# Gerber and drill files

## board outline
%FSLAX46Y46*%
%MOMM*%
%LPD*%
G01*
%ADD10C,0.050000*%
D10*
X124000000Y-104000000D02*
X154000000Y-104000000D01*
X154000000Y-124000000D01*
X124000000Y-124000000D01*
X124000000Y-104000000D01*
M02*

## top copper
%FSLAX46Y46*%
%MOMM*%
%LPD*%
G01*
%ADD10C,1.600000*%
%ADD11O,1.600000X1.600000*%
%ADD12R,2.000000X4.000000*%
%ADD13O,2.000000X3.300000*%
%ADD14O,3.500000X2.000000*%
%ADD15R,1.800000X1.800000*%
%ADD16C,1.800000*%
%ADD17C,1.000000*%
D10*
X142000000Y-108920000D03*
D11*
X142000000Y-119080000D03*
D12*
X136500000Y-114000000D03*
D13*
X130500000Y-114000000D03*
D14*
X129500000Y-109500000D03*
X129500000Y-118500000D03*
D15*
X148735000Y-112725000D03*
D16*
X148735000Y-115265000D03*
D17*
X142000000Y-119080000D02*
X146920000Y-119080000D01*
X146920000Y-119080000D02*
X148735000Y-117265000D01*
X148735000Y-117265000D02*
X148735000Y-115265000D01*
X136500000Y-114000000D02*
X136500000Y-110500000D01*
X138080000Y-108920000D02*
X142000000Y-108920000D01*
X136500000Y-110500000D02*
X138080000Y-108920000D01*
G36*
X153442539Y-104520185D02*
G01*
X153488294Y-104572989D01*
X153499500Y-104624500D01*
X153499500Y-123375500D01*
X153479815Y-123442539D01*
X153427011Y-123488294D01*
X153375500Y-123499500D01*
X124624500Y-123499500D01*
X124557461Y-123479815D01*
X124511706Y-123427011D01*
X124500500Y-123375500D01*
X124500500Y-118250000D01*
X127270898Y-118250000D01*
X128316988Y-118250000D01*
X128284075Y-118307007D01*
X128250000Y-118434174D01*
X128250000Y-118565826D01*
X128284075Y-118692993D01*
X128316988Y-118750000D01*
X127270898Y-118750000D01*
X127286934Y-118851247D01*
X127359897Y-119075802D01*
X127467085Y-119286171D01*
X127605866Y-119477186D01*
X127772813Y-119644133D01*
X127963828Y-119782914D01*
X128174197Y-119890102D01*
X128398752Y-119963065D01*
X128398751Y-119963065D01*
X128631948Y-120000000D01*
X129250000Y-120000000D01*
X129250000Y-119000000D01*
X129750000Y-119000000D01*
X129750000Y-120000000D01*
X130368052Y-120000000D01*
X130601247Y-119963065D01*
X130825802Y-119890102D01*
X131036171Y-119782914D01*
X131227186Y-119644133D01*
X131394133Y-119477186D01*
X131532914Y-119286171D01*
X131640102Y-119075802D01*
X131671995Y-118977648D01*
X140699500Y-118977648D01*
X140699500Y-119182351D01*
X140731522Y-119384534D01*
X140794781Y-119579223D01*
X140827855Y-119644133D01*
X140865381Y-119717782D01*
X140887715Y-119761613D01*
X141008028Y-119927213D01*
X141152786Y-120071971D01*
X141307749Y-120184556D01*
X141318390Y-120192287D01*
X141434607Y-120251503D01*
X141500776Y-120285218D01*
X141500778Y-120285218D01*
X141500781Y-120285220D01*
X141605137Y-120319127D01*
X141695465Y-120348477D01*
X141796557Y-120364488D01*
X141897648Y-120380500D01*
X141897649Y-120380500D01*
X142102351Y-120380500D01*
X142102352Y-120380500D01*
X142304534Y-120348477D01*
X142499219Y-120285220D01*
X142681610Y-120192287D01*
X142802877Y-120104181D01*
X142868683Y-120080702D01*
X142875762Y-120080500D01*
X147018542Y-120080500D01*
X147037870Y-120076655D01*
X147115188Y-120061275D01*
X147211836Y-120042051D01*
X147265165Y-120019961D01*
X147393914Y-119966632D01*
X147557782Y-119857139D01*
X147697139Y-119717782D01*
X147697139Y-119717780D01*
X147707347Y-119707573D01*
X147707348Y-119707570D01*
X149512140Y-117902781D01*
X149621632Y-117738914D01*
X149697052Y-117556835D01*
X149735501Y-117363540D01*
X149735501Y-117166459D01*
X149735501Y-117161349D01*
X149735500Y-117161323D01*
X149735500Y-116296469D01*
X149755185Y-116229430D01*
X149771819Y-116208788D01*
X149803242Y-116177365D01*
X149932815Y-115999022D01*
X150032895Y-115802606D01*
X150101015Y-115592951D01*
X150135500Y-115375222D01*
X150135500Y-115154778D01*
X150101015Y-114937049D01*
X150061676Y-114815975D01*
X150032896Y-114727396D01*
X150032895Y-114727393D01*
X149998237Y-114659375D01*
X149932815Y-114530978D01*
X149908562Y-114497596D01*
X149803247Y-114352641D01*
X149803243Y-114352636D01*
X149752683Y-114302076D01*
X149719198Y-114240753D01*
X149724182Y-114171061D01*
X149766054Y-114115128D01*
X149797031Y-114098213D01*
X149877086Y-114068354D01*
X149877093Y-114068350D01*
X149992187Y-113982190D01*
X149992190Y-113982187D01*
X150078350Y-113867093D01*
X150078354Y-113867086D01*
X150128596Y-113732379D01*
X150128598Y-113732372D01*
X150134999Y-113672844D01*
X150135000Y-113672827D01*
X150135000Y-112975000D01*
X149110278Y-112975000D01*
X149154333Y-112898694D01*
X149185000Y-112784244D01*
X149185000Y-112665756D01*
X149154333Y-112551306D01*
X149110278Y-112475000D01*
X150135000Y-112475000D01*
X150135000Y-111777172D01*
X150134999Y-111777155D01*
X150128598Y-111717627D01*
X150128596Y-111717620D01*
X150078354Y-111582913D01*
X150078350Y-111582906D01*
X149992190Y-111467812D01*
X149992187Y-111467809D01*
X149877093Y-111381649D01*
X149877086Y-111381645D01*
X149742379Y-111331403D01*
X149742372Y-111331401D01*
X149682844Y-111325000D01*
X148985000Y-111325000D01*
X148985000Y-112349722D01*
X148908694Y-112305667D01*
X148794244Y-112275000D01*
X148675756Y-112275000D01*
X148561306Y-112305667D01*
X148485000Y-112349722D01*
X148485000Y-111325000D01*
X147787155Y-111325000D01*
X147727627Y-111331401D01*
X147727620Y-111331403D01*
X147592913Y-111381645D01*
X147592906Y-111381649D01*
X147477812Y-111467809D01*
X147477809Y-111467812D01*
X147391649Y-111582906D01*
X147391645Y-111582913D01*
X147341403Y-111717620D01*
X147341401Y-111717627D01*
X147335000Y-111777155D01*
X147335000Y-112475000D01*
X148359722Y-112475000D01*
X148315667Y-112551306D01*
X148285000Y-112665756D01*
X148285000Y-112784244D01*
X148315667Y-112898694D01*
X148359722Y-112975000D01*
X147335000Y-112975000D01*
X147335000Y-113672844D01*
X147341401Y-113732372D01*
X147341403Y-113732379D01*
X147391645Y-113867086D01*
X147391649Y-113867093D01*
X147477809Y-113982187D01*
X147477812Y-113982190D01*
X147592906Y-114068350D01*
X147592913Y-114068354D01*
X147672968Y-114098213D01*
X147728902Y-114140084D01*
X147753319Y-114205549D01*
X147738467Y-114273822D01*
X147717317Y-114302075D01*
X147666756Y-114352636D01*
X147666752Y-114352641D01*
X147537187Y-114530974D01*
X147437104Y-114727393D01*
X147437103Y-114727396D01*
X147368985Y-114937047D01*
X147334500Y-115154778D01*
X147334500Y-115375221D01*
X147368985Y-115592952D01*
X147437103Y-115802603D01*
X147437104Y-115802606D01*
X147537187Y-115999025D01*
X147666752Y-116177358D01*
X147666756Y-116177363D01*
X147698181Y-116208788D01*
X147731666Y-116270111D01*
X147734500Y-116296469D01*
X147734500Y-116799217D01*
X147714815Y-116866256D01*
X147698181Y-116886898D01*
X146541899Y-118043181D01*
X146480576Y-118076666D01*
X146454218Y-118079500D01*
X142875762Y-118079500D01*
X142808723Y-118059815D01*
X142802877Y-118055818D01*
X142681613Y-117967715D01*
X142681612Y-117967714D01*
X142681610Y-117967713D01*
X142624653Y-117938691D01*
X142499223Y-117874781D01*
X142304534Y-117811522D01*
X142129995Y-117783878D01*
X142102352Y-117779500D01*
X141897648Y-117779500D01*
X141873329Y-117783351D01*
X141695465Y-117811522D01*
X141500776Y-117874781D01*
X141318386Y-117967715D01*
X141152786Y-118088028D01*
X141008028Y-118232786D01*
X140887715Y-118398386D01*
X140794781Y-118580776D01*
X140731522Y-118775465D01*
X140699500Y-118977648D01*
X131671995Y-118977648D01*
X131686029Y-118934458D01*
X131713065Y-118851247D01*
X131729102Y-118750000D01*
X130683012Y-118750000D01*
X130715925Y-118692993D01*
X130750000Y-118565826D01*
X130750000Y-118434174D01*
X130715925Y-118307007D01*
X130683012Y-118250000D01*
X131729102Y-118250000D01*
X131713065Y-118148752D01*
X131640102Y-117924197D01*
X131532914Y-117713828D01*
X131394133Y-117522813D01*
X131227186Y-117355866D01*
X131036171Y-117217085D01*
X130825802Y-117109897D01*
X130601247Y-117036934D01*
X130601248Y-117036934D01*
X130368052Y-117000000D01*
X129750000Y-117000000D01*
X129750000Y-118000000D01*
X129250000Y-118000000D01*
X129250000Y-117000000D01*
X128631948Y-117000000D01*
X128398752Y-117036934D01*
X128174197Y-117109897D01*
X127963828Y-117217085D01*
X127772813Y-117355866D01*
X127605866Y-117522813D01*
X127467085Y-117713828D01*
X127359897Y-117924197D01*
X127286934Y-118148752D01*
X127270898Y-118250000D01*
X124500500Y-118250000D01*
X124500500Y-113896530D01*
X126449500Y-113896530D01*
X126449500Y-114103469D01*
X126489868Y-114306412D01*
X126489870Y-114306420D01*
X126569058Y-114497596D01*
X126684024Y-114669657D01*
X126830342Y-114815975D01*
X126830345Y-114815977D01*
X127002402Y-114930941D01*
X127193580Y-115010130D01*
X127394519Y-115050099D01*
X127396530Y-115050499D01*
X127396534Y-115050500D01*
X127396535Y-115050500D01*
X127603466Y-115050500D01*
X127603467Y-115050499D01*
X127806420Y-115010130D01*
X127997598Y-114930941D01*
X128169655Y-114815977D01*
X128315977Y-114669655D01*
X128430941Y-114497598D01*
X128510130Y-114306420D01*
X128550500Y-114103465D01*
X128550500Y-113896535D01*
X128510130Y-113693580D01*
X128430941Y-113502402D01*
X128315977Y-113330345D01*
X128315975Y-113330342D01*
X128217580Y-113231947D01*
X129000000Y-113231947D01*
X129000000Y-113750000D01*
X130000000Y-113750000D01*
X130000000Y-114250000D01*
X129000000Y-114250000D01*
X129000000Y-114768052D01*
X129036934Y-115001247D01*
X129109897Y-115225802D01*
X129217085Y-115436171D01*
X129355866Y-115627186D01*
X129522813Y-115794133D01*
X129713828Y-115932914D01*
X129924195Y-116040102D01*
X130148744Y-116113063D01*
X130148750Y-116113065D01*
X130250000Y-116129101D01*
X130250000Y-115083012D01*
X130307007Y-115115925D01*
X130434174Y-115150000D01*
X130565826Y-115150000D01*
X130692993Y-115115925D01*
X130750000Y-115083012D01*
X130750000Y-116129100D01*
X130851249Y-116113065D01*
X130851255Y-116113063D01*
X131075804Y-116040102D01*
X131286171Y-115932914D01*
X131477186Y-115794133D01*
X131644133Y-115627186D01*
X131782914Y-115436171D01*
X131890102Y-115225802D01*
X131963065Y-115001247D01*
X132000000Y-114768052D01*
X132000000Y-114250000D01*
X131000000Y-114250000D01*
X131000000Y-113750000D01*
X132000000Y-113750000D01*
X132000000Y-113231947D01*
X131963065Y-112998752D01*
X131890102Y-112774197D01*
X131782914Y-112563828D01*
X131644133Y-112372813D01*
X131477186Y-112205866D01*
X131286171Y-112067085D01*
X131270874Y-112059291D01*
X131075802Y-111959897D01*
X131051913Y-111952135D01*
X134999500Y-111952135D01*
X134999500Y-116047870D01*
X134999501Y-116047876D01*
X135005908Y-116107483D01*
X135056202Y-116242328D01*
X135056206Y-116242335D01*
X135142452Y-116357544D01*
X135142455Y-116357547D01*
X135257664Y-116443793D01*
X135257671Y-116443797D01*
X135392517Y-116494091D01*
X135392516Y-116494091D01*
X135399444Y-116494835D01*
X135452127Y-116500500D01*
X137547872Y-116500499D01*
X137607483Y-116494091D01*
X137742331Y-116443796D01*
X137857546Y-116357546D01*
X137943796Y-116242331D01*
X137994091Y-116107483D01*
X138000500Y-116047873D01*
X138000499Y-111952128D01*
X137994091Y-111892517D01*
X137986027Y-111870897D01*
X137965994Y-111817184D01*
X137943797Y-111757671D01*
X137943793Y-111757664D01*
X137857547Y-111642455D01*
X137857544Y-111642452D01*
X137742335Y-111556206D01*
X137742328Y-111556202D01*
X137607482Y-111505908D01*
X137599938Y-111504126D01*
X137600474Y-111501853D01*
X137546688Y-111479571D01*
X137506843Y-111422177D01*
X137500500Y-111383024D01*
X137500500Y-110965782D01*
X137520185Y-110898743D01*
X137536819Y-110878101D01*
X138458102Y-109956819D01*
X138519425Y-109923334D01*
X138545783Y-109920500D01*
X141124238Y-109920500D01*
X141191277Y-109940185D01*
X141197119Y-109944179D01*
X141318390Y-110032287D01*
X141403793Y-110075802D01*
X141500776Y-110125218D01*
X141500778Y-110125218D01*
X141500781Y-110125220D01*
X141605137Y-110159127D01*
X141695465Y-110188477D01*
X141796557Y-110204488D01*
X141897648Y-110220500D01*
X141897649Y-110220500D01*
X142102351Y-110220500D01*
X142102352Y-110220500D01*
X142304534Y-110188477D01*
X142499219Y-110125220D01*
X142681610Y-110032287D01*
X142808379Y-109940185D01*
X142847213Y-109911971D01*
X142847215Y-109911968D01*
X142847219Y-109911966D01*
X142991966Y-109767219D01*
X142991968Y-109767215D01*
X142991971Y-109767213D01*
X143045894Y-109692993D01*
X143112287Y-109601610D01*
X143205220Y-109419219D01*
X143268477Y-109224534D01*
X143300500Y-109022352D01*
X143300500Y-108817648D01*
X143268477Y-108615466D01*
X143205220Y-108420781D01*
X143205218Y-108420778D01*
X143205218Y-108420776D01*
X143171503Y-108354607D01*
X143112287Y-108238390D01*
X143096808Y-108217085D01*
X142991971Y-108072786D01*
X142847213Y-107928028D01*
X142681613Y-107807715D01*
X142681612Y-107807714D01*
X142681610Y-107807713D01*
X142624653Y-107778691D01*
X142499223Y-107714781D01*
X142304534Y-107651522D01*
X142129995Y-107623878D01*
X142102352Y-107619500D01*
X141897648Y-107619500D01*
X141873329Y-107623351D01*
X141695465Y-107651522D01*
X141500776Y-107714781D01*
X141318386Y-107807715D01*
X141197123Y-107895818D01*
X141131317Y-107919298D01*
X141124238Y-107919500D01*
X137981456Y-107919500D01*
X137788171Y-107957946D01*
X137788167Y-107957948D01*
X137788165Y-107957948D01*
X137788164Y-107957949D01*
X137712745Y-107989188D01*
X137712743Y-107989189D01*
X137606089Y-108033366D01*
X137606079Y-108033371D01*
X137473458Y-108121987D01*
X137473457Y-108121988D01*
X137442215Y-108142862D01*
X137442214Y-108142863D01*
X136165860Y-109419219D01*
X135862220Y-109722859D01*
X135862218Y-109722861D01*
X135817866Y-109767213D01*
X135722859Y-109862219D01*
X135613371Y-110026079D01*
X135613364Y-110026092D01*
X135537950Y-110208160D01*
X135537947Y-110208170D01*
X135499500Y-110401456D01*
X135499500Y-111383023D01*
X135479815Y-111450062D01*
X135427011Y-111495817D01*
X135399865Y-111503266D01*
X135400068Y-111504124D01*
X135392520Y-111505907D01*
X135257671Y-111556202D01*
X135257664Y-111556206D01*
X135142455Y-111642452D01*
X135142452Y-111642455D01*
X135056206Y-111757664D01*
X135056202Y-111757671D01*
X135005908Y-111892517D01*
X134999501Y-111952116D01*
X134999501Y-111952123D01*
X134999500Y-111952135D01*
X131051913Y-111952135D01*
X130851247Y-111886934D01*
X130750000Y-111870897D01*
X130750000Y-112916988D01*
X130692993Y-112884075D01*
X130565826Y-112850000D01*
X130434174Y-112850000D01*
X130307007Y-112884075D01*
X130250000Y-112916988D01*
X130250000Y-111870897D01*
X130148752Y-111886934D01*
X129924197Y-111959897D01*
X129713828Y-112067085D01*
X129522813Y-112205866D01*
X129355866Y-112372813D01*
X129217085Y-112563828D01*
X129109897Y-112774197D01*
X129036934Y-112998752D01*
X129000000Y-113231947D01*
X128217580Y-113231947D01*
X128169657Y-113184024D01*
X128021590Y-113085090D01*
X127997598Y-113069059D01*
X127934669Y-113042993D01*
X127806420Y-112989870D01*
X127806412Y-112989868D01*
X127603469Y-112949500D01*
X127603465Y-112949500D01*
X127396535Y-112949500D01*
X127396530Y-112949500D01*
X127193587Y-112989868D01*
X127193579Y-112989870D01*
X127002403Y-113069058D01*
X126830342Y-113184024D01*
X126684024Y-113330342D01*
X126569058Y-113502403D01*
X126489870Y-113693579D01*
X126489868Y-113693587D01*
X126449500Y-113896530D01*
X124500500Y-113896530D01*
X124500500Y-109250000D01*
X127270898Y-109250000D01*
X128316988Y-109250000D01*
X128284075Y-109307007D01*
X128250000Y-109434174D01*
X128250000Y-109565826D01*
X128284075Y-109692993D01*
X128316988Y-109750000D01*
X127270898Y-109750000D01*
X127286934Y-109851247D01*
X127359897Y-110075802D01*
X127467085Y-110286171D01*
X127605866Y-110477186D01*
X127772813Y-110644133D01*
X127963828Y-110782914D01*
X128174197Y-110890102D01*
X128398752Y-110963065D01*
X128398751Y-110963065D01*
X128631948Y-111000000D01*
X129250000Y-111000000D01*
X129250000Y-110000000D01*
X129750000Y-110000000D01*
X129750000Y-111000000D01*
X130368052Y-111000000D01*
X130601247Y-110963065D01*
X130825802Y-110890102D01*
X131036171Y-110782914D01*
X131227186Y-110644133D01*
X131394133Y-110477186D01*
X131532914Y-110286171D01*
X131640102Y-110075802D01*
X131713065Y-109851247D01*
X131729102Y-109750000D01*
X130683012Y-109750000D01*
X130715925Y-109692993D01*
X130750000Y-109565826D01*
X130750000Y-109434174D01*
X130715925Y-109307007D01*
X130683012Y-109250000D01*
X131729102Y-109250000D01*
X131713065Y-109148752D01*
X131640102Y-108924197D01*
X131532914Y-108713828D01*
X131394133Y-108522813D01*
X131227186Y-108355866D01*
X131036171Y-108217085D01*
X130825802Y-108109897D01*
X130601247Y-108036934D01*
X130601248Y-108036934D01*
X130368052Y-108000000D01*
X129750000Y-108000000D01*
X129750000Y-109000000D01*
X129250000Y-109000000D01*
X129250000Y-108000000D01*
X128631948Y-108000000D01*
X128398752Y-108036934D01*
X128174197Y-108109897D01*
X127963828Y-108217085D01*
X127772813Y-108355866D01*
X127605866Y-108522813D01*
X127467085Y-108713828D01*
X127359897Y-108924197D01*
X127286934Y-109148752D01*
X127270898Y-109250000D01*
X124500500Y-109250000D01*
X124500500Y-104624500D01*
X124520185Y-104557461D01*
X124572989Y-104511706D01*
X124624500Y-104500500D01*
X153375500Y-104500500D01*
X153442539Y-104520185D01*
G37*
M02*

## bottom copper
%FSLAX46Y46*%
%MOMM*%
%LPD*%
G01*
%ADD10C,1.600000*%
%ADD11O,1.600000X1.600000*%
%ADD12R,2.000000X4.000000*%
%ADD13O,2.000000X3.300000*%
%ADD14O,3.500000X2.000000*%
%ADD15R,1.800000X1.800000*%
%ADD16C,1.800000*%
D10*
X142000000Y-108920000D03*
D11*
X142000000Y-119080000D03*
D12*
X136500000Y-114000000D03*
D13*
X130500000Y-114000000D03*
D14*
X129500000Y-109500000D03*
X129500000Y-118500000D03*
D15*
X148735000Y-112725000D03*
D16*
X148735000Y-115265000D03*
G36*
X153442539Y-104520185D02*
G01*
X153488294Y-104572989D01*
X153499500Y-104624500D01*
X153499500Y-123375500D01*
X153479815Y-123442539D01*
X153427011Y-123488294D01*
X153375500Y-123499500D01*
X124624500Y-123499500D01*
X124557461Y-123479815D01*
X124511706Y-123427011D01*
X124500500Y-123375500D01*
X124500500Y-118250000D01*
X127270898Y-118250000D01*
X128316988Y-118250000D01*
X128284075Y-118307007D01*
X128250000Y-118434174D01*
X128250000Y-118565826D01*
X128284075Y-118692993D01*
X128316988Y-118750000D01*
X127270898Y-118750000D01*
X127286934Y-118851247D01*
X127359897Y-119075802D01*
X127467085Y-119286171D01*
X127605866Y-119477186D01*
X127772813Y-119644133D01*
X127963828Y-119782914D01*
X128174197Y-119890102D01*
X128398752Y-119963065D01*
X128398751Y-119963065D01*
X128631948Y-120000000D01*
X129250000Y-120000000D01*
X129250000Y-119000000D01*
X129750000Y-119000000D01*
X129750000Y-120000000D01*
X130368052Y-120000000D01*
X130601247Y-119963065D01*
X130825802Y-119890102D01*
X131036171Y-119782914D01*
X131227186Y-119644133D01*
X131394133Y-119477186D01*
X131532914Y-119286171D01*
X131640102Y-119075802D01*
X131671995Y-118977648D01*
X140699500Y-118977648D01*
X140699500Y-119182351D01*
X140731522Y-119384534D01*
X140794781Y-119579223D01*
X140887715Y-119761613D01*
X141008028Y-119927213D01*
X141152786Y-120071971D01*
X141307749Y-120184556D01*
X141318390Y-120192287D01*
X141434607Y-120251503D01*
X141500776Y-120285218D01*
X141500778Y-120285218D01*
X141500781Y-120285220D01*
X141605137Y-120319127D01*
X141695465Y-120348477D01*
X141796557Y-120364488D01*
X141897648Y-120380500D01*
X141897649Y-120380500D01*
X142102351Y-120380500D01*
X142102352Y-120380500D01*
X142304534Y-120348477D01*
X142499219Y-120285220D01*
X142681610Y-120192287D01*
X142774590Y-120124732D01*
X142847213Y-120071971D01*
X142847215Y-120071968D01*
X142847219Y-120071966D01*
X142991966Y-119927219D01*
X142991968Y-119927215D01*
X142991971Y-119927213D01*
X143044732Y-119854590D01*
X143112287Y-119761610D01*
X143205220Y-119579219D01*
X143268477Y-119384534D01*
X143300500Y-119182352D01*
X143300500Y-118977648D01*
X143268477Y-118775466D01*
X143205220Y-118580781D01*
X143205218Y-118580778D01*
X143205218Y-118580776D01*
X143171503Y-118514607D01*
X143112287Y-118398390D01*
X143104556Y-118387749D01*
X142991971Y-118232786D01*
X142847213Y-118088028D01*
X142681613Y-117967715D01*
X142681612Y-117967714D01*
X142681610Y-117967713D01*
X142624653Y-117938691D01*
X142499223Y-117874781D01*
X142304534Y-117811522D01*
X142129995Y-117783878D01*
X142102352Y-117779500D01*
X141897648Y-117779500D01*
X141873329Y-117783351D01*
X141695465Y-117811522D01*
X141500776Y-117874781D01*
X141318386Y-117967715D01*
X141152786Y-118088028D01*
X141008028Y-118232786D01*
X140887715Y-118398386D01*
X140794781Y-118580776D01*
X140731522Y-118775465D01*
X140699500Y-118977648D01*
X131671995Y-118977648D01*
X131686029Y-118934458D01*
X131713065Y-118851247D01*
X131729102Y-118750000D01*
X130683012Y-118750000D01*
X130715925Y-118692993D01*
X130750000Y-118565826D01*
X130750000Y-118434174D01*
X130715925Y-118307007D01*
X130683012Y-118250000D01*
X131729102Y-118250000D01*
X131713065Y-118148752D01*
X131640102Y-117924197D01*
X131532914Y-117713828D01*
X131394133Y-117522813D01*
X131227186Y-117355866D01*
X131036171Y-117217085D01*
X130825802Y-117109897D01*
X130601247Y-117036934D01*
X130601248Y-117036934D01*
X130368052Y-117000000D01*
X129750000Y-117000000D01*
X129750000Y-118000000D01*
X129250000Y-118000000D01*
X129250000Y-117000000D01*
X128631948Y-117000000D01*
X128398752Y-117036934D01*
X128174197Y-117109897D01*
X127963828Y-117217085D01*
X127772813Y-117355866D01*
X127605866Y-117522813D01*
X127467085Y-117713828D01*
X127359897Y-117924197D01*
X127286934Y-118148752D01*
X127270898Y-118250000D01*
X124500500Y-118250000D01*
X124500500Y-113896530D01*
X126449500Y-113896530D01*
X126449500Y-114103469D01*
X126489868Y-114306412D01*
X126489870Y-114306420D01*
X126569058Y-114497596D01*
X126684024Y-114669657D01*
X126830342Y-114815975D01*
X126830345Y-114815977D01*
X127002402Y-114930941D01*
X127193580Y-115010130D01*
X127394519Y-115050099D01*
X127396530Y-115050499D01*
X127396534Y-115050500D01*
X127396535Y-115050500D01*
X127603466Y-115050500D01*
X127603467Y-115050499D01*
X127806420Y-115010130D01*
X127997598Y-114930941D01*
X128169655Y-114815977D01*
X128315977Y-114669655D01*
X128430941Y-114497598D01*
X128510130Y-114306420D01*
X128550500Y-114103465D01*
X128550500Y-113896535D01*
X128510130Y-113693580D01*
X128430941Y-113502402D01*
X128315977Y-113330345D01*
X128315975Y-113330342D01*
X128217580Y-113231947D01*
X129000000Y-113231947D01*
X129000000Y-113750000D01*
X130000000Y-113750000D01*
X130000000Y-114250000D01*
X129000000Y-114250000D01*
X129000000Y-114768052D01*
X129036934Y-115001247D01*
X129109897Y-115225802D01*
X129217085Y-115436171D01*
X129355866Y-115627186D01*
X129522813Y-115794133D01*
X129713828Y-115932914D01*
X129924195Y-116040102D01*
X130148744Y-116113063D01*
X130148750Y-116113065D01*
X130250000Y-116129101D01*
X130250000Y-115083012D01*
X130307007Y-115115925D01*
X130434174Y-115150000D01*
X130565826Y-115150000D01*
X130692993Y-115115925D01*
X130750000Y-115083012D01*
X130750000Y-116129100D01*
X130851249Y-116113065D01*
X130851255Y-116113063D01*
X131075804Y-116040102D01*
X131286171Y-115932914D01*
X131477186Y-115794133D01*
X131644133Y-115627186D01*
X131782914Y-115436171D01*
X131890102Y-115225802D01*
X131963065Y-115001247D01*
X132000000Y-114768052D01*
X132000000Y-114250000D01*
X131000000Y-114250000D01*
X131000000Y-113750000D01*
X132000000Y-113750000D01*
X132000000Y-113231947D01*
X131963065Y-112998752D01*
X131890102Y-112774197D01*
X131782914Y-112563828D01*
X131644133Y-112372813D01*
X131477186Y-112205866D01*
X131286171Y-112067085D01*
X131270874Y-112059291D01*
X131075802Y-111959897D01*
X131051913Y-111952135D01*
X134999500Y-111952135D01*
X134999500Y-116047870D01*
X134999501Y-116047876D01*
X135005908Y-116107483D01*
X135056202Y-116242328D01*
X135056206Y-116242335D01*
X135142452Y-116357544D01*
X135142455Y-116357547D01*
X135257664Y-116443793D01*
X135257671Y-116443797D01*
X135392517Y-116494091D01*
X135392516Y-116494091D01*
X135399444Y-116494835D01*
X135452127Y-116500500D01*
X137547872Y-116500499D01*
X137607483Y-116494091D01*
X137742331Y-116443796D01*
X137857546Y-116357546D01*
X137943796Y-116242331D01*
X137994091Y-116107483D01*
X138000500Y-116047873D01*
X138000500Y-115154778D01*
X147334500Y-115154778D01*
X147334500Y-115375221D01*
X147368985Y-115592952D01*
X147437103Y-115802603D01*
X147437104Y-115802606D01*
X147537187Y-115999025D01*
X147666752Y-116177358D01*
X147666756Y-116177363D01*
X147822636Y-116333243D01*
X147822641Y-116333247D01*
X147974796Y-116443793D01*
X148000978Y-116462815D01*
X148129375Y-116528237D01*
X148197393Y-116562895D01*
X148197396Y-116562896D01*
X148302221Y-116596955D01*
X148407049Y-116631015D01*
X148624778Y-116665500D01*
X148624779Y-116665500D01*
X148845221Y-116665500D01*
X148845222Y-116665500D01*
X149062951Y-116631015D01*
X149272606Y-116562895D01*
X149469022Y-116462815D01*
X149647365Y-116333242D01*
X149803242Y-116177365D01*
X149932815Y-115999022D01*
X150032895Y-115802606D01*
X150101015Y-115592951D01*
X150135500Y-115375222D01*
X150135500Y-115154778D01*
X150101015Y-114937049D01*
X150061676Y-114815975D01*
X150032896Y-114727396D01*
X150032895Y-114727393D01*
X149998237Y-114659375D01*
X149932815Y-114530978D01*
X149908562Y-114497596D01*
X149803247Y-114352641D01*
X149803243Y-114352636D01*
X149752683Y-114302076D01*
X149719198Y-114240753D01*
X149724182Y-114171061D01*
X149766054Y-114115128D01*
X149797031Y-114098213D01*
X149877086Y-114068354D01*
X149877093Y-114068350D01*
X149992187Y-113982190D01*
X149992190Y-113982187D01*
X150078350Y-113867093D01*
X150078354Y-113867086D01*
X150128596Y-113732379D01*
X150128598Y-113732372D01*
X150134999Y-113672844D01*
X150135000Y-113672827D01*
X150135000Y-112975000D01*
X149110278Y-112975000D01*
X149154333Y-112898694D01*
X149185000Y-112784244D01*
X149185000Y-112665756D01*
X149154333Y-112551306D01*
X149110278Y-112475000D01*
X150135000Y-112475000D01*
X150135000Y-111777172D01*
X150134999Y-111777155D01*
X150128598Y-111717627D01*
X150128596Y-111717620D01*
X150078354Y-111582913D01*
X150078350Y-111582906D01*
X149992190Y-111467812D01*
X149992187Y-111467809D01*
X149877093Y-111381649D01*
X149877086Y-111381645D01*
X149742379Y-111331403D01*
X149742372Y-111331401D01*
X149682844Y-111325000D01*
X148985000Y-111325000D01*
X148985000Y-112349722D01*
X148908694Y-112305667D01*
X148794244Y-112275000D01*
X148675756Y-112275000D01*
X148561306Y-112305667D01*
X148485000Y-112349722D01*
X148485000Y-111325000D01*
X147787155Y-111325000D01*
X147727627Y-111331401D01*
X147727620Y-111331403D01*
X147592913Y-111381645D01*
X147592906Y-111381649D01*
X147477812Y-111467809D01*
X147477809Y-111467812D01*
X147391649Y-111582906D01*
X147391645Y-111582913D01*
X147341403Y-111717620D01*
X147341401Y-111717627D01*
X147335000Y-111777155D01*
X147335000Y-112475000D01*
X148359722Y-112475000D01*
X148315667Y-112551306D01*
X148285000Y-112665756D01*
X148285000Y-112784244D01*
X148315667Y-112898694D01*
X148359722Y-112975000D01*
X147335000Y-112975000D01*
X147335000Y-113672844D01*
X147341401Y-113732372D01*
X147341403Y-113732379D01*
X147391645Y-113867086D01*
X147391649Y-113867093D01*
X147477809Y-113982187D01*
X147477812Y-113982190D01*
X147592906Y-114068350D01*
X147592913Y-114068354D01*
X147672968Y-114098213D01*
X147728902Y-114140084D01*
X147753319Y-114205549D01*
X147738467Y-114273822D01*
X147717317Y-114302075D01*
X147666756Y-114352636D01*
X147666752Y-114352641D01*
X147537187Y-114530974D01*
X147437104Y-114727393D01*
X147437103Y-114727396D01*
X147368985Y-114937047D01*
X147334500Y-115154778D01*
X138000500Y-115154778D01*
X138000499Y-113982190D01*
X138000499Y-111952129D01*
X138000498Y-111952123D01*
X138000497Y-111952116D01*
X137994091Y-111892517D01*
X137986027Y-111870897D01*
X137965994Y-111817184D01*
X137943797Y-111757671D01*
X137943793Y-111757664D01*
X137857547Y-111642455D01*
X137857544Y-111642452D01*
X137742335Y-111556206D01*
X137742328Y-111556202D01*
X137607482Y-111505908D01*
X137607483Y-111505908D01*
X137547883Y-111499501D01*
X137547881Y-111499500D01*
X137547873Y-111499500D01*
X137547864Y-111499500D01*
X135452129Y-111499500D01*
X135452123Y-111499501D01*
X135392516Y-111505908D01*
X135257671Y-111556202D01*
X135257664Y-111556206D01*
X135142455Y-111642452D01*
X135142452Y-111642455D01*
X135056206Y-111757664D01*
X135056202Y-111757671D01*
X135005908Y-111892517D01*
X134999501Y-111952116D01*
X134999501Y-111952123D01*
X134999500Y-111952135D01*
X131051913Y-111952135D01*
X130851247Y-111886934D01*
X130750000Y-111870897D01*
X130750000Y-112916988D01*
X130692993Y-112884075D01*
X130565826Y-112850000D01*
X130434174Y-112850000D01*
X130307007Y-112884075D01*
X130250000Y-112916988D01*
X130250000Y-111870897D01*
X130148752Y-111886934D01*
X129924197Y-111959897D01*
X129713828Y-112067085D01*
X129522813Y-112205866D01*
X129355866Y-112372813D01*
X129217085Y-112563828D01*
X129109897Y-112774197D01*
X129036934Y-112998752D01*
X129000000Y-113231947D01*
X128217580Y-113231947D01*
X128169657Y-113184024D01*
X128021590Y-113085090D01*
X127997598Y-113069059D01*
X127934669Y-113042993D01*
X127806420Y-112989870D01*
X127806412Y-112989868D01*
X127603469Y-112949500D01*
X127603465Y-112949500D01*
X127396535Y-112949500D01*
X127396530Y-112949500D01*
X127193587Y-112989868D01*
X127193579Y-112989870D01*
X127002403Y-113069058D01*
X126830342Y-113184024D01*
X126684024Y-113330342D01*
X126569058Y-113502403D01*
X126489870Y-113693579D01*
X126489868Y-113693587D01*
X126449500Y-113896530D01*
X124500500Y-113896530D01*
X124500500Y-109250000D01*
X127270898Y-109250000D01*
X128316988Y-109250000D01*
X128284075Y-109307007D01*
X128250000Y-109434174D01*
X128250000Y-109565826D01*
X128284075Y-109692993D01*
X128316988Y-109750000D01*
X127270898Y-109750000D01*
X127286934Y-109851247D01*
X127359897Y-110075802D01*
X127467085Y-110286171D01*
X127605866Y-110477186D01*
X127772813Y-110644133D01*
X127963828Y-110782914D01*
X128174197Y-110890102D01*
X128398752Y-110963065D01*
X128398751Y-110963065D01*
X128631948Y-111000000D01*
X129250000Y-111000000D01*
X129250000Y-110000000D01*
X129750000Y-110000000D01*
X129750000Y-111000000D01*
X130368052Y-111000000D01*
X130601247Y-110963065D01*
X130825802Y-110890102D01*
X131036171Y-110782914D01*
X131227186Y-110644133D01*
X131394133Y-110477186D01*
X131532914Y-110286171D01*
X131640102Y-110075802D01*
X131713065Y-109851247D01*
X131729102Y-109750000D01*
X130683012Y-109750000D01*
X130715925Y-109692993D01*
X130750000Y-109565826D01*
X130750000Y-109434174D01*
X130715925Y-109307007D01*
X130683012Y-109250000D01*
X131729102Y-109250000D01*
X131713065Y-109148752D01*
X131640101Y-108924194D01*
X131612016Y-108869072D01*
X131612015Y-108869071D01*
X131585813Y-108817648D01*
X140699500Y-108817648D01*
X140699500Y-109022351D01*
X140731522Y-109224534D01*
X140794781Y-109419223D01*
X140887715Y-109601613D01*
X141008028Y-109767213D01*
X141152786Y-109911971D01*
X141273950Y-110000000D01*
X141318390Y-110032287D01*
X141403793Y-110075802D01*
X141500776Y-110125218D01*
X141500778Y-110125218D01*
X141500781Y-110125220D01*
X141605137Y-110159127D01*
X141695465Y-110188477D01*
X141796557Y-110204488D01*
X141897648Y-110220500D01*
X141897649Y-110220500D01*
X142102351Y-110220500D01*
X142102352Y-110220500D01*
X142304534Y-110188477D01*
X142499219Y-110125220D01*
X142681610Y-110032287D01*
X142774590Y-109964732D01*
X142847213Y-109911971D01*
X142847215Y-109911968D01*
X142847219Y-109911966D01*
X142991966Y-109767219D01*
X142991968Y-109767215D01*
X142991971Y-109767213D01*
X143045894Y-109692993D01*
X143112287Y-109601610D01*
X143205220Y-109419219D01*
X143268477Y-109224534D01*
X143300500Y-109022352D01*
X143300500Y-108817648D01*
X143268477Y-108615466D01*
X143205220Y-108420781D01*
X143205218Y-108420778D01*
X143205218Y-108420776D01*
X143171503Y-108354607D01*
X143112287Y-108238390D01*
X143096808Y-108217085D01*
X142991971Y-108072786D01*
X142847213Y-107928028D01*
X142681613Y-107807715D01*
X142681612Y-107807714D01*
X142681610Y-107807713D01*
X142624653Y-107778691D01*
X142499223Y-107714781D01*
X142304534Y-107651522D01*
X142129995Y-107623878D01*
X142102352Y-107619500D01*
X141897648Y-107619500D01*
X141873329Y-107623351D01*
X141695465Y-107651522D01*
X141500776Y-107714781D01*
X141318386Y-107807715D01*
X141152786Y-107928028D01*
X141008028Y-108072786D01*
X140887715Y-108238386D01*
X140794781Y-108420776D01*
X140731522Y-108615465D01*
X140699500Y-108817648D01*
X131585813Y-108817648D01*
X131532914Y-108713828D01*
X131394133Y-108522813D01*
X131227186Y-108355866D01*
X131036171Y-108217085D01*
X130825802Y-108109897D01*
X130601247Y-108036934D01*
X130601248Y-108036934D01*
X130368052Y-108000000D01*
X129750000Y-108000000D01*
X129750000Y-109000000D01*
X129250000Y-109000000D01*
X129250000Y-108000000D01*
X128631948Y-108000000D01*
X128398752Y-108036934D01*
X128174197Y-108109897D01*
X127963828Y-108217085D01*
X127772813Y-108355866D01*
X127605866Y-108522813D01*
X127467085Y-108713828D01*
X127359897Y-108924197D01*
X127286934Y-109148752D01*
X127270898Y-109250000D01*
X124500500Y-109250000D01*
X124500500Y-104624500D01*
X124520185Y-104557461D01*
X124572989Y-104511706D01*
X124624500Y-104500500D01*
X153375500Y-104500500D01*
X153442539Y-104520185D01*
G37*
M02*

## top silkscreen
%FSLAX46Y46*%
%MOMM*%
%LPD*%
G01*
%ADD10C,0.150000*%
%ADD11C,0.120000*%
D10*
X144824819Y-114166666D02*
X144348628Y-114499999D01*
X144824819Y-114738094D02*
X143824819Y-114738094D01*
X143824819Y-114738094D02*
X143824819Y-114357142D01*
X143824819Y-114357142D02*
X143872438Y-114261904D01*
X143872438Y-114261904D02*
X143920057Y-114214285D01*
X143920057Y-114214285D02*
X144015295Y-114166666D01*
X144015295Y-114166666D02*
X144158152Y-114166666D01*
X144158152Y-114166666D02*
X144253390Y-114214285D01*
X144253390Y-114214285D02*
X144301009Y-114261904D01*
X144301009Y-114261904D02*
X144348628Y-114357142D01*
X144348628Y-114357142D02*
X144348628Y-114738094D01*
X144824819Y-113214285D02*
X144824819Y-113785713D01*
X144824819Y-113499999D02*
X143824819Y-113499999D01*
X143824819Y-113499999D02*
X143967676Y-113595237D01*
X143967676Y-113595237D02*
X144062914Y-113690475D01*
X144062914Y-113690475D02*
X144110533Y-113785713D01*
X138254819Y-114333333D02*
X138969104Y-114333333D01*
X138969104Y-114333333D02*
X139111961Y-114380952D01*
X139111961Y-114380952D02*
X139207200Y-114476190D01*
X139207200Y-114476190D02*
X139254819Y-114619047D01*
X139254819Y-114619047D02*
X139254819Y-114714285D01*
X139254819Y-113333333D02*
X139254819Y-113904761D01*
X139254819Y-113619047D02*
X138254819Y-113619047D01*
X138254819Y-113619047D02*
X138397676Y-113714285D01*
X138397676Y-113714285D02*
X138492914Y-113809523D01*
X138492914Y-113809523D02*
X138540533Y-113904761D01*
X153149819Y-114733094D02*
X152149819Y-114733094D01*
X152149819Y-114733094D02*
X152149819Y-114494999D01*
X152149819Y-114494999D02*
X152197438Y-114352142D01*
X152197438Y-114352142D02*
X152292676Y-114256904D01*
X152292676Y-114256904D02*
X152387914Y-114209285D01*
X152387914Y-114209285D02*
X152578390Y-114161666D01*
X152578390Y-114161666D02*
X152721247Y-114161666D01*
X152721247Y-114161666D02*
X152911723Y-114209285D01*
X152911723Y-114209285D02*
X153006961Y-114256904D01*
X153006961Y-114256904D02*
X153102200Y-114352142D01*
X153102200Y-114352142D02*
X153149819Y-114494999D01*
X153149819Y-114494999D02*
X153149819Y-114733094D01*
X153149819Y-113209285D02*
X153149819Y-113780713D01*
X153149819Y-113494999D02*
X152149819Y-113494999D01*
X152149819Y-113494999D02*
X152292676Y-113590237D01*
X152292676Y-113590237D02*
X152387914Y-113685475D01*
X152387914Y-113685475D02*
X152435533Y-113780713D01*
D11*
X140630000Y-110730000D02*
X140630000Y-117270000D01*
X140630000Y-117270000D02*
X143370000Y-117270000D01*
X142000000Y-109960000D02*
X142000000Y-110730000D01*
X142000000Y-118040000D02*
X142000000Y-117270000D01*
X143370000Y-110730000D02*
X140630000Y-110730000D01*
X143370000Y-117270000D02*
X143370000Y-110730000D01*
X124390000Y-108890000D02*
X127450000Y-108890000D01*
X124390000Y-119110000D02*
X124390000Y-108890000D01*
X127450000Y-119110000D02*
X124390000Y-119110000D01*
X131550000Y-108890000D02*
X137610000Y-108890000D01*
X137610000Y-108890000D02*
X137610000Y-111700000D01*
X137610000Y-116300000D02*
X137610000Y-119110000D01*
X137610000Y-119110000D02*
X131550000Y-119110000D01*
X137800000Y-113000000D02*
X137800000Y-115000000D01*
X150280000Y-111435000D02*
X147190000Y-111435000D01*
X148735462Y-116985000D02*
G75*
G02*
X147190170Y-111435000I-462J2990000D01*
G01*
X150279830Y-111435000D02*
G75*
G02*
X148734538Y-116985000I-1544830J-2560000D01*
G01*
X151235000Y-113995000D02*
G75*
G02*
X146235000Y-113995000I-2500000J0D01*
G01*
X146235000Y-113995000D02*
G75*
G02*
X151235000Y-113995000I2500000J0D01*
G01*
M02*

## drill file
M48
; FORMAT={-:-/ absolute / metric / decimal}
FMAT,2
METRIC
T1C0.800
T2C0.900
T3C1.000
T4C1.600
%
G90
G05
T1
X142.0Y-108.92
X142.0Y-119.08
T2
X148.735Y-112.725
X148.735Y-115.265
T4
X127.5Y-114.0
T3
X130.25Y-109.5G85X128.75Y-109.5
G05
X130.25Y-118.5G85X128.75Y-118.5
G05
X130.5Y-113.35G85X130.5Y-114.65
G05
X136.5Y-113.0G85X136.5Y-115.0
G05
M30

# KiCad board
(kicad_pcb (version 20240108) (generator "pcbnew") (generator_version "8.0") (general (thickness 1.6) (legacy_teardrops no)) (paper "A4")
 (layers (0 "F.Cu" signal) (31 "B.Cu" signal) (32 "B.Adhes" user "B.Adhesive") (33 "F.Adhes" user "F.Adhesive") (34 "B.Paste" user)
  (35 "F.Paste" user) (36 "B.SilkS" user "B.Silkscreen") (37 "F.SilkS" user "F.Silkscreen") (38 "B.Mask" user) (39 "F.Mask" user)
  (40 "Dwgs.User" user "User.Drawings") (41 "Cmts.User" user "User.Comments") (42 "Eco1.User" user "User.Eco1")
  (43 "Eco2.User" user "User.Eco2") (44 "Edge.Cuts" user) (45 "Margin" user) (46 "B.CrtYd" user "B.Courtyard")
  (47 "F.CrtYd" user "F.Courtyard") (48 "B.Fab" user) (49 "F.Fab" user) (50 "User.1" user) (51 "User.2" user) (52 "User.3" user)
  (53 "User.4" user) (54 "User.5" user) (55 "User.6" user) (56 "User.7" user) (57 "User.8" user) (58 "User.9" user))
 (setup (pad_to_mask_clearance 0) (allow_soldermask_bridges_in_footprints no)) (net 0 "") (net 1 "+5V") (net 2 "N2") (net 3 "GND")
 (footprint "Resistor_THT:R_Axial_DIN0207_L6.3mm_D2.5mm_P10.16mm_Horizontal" (layer "F.Cu") (at 142 108.92 -90)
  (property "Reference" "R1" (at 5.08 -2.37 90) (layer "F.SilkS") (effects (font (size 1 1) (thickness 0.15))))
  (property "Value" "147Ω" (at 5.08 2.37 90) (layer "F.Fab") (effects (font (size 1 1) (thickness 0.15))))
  (fp_line (start 1.81 1.37) (end 8.35 1.37) (stroke (width 0.12) (type solid)) (layer "F.SilkS"))
  (fp_line (start 8.35 1.37) (end 8.35 -1.37) (stroke (width 0.12) (type solid)) (layer "F.SilkS"))
  (fp_line (start 1.04 0) (end 1.81 0) (stroke (width 0.12) (type solid)) (layer "F.SilkS"))
  (fp_line (start 9.12 0) (end 8.35 0) (stroke (width 0.12) (type solid)) (layer "F.SilkS"))
  (fp_line (start 1.81 -1.37) (end 1.81 1.37) (stroke (width 0.12) (type solid)) (layer "F.SilkS"))
  (fp_line (start 8.35 -1.37) (end 1.81 -1.37) (stroke (width 0.12) (type solid)) (layer "F.SilkS"))
  (pad "1" thru_hole circle (at 0 0 270) (size 1.6 1.6) (drill 0.8) (layers "*.Cu" "*.Mask") (remove_unused_layers no) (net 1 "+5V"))
  (pad "2" thru_hole oval (at 10.16 0 270) (size 1.6 1.6) (drill 0.8) (layers "*.Cu" "*.Mask") (remove_unused_layers no) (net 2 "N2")))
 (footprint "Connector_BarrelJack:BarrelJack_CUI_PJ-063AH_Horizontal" (layer "F.Cu") (at 136.5 114 -90)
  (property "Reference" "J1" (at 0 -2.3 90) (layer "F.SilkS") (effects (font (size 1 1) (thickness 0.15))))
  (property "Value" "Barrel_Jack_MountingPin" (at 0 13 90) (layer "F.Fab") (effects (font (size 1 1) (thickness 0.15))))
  (fp_line (start -5.11 12.11) (end -5.11 9.05) (stroke (width 0.12) (type solid)) (layer "F.SilkS"))
  (fp_line (start 5.11 12.11) (end -5.11 12.11) (stroke (width 0.12) (type solid)) (layer "F.SilkS"))
  (fp_line (start 5.11 9.05) (end 5.11 12.11) (stroke (width 0.12) (type solid)) (layer "F.SilkS"))
  (fp_line (start -5.11 4.95) (end -5.11 -1.11) (stroke (width 0.12) (type solid)) (layer "F.SilkS"))
  (fp_line (start -5.11 -1.11) (end -2.3 -1.11) (stroke (width 0.12) (type solid)) (layer "F.SilkS"))
  (fp_line (start 2.3 -1.11) (end 5.11 -1.11) (stroke (width 0.12) (type solid)) (layer "F.SilkS"))
  (fp_line (start 5.11 -1.11) (end 5.11 4.95) (stroke (width 0.12) (type solid)) (layer "F.SilkS"))
  (fp_line (start -1 -1.3) (end 1 -1.3) (stroke (width 0.12) (type solid)) (layer "F.SilkS"))
  (pad "" np_thru_hole circle (at 0 9 270) (size 1.6 1.6) (drill 1.6) (layers "*.Cu" "*.Mask"))
  (pad "1" thru_hole rect (at 0 0 270) (size 4 2) (drill oval 3 1) (layers "*.Cu" "*.Mask") (remove_unused_layers no) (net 1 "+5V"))
  (pad "2" thru_hole oval (at 0 6 270) (size 3.3 2) (drill oval 2.3 1) (layers "*.Cu" "*.Mask") (remove_unused_layers no) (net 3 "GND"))
  (pad "MP" thru_hole oval (at -4.5 7 270) (size 2 3.5) (drill oval 1 2.5) (layers "*.Cu" "*.Mask") (remove_unused_layers no) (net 3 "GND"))
  (pad "MP" thru_hole oval (at 4.5 7 270) (size 2 3.5) (drill oval 1 2.5) (layers "*.Cu" "*.Mask") (remove_unused_layers no) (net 3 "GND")))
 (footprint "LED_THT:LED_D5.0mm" (layer "F.Cu") (at 148.735 112.725 -90)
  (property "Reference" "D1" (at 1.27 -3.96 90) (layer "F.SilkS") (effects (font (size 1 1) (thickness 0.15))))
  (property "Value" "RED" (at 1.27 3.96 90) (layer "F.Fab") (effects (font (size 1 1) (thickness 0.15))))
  (fp_line (start -1.29 -1.545) (end -1.29 1.545) (stroke (width 0.12) (type solid)) (layer "F.SilkS"))
  (fp_arc (start 4.26 -0.000462) (mid 2.072002 2.880433) (end -1.29 1.54483) (stroke (width 0.12) (type solid)) (layer "F.SilkS"))
  (fp_arc (start -1.29 -1.54483) (mid 2.072002 -2.880433) (end 4.26 0.000462) (stroke (width 0.12) (type solid)) (layer "F.SilkS"))
  (fp_circle (center 1.27 0) (end 3.77 0) (stroke (width 0.12) (type solid)) (fill none) (layer "F.SilkS"))
  (pad "1" thru_hole rect (at 0 0 270) (size 1.8 1.8) (drill 0.9) (layers "*.Cu" "*.Mask") (remove_unused_layers no) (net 3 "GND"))
  (pad "2" thru_hole circle (at 2.54 0 270) (size 1.8 1.8) (drill 0.9) (layers "*.Cu" "*.Mask") (remove_unused_layers no) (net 2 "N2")))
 (gr_rect (start 124 104) (end 154 124) (stroke (width 0.05) (type default)) (fill none) (layer "Edge.Cuts"))
 (segment (start 142 119.08) (end 146.92 119.08) (width 1) (layer "F.Cu") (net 2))
 (segment (start 146.92 119.08) (end 148.735 117.265) (width 1) (layer "F.Cu") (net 2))
 (segment (start 148.735 117.265) (end 148.735 115.265) (width 1) (layer "F.Cu") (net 2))
 (segment (start 136.5 114) (end 136.5 110.5) (width 1) (layer "F.Cu") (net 1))
 (segment (start 138.08 108.92) (end 142 108.92) (width 1) (layer "F.Cu") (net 1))
 (segment (start 136.5 110.5) (end 138.08 108.92) (width 1) (layer "F.Cu") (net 1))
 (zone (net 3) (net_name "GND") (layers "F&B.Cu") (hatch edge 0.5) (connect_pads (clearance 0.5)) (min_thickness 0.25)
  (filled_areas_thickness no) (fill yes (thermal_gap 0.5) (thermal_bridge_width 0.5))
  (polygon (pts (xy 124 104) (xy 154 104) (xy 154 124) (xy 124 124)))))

